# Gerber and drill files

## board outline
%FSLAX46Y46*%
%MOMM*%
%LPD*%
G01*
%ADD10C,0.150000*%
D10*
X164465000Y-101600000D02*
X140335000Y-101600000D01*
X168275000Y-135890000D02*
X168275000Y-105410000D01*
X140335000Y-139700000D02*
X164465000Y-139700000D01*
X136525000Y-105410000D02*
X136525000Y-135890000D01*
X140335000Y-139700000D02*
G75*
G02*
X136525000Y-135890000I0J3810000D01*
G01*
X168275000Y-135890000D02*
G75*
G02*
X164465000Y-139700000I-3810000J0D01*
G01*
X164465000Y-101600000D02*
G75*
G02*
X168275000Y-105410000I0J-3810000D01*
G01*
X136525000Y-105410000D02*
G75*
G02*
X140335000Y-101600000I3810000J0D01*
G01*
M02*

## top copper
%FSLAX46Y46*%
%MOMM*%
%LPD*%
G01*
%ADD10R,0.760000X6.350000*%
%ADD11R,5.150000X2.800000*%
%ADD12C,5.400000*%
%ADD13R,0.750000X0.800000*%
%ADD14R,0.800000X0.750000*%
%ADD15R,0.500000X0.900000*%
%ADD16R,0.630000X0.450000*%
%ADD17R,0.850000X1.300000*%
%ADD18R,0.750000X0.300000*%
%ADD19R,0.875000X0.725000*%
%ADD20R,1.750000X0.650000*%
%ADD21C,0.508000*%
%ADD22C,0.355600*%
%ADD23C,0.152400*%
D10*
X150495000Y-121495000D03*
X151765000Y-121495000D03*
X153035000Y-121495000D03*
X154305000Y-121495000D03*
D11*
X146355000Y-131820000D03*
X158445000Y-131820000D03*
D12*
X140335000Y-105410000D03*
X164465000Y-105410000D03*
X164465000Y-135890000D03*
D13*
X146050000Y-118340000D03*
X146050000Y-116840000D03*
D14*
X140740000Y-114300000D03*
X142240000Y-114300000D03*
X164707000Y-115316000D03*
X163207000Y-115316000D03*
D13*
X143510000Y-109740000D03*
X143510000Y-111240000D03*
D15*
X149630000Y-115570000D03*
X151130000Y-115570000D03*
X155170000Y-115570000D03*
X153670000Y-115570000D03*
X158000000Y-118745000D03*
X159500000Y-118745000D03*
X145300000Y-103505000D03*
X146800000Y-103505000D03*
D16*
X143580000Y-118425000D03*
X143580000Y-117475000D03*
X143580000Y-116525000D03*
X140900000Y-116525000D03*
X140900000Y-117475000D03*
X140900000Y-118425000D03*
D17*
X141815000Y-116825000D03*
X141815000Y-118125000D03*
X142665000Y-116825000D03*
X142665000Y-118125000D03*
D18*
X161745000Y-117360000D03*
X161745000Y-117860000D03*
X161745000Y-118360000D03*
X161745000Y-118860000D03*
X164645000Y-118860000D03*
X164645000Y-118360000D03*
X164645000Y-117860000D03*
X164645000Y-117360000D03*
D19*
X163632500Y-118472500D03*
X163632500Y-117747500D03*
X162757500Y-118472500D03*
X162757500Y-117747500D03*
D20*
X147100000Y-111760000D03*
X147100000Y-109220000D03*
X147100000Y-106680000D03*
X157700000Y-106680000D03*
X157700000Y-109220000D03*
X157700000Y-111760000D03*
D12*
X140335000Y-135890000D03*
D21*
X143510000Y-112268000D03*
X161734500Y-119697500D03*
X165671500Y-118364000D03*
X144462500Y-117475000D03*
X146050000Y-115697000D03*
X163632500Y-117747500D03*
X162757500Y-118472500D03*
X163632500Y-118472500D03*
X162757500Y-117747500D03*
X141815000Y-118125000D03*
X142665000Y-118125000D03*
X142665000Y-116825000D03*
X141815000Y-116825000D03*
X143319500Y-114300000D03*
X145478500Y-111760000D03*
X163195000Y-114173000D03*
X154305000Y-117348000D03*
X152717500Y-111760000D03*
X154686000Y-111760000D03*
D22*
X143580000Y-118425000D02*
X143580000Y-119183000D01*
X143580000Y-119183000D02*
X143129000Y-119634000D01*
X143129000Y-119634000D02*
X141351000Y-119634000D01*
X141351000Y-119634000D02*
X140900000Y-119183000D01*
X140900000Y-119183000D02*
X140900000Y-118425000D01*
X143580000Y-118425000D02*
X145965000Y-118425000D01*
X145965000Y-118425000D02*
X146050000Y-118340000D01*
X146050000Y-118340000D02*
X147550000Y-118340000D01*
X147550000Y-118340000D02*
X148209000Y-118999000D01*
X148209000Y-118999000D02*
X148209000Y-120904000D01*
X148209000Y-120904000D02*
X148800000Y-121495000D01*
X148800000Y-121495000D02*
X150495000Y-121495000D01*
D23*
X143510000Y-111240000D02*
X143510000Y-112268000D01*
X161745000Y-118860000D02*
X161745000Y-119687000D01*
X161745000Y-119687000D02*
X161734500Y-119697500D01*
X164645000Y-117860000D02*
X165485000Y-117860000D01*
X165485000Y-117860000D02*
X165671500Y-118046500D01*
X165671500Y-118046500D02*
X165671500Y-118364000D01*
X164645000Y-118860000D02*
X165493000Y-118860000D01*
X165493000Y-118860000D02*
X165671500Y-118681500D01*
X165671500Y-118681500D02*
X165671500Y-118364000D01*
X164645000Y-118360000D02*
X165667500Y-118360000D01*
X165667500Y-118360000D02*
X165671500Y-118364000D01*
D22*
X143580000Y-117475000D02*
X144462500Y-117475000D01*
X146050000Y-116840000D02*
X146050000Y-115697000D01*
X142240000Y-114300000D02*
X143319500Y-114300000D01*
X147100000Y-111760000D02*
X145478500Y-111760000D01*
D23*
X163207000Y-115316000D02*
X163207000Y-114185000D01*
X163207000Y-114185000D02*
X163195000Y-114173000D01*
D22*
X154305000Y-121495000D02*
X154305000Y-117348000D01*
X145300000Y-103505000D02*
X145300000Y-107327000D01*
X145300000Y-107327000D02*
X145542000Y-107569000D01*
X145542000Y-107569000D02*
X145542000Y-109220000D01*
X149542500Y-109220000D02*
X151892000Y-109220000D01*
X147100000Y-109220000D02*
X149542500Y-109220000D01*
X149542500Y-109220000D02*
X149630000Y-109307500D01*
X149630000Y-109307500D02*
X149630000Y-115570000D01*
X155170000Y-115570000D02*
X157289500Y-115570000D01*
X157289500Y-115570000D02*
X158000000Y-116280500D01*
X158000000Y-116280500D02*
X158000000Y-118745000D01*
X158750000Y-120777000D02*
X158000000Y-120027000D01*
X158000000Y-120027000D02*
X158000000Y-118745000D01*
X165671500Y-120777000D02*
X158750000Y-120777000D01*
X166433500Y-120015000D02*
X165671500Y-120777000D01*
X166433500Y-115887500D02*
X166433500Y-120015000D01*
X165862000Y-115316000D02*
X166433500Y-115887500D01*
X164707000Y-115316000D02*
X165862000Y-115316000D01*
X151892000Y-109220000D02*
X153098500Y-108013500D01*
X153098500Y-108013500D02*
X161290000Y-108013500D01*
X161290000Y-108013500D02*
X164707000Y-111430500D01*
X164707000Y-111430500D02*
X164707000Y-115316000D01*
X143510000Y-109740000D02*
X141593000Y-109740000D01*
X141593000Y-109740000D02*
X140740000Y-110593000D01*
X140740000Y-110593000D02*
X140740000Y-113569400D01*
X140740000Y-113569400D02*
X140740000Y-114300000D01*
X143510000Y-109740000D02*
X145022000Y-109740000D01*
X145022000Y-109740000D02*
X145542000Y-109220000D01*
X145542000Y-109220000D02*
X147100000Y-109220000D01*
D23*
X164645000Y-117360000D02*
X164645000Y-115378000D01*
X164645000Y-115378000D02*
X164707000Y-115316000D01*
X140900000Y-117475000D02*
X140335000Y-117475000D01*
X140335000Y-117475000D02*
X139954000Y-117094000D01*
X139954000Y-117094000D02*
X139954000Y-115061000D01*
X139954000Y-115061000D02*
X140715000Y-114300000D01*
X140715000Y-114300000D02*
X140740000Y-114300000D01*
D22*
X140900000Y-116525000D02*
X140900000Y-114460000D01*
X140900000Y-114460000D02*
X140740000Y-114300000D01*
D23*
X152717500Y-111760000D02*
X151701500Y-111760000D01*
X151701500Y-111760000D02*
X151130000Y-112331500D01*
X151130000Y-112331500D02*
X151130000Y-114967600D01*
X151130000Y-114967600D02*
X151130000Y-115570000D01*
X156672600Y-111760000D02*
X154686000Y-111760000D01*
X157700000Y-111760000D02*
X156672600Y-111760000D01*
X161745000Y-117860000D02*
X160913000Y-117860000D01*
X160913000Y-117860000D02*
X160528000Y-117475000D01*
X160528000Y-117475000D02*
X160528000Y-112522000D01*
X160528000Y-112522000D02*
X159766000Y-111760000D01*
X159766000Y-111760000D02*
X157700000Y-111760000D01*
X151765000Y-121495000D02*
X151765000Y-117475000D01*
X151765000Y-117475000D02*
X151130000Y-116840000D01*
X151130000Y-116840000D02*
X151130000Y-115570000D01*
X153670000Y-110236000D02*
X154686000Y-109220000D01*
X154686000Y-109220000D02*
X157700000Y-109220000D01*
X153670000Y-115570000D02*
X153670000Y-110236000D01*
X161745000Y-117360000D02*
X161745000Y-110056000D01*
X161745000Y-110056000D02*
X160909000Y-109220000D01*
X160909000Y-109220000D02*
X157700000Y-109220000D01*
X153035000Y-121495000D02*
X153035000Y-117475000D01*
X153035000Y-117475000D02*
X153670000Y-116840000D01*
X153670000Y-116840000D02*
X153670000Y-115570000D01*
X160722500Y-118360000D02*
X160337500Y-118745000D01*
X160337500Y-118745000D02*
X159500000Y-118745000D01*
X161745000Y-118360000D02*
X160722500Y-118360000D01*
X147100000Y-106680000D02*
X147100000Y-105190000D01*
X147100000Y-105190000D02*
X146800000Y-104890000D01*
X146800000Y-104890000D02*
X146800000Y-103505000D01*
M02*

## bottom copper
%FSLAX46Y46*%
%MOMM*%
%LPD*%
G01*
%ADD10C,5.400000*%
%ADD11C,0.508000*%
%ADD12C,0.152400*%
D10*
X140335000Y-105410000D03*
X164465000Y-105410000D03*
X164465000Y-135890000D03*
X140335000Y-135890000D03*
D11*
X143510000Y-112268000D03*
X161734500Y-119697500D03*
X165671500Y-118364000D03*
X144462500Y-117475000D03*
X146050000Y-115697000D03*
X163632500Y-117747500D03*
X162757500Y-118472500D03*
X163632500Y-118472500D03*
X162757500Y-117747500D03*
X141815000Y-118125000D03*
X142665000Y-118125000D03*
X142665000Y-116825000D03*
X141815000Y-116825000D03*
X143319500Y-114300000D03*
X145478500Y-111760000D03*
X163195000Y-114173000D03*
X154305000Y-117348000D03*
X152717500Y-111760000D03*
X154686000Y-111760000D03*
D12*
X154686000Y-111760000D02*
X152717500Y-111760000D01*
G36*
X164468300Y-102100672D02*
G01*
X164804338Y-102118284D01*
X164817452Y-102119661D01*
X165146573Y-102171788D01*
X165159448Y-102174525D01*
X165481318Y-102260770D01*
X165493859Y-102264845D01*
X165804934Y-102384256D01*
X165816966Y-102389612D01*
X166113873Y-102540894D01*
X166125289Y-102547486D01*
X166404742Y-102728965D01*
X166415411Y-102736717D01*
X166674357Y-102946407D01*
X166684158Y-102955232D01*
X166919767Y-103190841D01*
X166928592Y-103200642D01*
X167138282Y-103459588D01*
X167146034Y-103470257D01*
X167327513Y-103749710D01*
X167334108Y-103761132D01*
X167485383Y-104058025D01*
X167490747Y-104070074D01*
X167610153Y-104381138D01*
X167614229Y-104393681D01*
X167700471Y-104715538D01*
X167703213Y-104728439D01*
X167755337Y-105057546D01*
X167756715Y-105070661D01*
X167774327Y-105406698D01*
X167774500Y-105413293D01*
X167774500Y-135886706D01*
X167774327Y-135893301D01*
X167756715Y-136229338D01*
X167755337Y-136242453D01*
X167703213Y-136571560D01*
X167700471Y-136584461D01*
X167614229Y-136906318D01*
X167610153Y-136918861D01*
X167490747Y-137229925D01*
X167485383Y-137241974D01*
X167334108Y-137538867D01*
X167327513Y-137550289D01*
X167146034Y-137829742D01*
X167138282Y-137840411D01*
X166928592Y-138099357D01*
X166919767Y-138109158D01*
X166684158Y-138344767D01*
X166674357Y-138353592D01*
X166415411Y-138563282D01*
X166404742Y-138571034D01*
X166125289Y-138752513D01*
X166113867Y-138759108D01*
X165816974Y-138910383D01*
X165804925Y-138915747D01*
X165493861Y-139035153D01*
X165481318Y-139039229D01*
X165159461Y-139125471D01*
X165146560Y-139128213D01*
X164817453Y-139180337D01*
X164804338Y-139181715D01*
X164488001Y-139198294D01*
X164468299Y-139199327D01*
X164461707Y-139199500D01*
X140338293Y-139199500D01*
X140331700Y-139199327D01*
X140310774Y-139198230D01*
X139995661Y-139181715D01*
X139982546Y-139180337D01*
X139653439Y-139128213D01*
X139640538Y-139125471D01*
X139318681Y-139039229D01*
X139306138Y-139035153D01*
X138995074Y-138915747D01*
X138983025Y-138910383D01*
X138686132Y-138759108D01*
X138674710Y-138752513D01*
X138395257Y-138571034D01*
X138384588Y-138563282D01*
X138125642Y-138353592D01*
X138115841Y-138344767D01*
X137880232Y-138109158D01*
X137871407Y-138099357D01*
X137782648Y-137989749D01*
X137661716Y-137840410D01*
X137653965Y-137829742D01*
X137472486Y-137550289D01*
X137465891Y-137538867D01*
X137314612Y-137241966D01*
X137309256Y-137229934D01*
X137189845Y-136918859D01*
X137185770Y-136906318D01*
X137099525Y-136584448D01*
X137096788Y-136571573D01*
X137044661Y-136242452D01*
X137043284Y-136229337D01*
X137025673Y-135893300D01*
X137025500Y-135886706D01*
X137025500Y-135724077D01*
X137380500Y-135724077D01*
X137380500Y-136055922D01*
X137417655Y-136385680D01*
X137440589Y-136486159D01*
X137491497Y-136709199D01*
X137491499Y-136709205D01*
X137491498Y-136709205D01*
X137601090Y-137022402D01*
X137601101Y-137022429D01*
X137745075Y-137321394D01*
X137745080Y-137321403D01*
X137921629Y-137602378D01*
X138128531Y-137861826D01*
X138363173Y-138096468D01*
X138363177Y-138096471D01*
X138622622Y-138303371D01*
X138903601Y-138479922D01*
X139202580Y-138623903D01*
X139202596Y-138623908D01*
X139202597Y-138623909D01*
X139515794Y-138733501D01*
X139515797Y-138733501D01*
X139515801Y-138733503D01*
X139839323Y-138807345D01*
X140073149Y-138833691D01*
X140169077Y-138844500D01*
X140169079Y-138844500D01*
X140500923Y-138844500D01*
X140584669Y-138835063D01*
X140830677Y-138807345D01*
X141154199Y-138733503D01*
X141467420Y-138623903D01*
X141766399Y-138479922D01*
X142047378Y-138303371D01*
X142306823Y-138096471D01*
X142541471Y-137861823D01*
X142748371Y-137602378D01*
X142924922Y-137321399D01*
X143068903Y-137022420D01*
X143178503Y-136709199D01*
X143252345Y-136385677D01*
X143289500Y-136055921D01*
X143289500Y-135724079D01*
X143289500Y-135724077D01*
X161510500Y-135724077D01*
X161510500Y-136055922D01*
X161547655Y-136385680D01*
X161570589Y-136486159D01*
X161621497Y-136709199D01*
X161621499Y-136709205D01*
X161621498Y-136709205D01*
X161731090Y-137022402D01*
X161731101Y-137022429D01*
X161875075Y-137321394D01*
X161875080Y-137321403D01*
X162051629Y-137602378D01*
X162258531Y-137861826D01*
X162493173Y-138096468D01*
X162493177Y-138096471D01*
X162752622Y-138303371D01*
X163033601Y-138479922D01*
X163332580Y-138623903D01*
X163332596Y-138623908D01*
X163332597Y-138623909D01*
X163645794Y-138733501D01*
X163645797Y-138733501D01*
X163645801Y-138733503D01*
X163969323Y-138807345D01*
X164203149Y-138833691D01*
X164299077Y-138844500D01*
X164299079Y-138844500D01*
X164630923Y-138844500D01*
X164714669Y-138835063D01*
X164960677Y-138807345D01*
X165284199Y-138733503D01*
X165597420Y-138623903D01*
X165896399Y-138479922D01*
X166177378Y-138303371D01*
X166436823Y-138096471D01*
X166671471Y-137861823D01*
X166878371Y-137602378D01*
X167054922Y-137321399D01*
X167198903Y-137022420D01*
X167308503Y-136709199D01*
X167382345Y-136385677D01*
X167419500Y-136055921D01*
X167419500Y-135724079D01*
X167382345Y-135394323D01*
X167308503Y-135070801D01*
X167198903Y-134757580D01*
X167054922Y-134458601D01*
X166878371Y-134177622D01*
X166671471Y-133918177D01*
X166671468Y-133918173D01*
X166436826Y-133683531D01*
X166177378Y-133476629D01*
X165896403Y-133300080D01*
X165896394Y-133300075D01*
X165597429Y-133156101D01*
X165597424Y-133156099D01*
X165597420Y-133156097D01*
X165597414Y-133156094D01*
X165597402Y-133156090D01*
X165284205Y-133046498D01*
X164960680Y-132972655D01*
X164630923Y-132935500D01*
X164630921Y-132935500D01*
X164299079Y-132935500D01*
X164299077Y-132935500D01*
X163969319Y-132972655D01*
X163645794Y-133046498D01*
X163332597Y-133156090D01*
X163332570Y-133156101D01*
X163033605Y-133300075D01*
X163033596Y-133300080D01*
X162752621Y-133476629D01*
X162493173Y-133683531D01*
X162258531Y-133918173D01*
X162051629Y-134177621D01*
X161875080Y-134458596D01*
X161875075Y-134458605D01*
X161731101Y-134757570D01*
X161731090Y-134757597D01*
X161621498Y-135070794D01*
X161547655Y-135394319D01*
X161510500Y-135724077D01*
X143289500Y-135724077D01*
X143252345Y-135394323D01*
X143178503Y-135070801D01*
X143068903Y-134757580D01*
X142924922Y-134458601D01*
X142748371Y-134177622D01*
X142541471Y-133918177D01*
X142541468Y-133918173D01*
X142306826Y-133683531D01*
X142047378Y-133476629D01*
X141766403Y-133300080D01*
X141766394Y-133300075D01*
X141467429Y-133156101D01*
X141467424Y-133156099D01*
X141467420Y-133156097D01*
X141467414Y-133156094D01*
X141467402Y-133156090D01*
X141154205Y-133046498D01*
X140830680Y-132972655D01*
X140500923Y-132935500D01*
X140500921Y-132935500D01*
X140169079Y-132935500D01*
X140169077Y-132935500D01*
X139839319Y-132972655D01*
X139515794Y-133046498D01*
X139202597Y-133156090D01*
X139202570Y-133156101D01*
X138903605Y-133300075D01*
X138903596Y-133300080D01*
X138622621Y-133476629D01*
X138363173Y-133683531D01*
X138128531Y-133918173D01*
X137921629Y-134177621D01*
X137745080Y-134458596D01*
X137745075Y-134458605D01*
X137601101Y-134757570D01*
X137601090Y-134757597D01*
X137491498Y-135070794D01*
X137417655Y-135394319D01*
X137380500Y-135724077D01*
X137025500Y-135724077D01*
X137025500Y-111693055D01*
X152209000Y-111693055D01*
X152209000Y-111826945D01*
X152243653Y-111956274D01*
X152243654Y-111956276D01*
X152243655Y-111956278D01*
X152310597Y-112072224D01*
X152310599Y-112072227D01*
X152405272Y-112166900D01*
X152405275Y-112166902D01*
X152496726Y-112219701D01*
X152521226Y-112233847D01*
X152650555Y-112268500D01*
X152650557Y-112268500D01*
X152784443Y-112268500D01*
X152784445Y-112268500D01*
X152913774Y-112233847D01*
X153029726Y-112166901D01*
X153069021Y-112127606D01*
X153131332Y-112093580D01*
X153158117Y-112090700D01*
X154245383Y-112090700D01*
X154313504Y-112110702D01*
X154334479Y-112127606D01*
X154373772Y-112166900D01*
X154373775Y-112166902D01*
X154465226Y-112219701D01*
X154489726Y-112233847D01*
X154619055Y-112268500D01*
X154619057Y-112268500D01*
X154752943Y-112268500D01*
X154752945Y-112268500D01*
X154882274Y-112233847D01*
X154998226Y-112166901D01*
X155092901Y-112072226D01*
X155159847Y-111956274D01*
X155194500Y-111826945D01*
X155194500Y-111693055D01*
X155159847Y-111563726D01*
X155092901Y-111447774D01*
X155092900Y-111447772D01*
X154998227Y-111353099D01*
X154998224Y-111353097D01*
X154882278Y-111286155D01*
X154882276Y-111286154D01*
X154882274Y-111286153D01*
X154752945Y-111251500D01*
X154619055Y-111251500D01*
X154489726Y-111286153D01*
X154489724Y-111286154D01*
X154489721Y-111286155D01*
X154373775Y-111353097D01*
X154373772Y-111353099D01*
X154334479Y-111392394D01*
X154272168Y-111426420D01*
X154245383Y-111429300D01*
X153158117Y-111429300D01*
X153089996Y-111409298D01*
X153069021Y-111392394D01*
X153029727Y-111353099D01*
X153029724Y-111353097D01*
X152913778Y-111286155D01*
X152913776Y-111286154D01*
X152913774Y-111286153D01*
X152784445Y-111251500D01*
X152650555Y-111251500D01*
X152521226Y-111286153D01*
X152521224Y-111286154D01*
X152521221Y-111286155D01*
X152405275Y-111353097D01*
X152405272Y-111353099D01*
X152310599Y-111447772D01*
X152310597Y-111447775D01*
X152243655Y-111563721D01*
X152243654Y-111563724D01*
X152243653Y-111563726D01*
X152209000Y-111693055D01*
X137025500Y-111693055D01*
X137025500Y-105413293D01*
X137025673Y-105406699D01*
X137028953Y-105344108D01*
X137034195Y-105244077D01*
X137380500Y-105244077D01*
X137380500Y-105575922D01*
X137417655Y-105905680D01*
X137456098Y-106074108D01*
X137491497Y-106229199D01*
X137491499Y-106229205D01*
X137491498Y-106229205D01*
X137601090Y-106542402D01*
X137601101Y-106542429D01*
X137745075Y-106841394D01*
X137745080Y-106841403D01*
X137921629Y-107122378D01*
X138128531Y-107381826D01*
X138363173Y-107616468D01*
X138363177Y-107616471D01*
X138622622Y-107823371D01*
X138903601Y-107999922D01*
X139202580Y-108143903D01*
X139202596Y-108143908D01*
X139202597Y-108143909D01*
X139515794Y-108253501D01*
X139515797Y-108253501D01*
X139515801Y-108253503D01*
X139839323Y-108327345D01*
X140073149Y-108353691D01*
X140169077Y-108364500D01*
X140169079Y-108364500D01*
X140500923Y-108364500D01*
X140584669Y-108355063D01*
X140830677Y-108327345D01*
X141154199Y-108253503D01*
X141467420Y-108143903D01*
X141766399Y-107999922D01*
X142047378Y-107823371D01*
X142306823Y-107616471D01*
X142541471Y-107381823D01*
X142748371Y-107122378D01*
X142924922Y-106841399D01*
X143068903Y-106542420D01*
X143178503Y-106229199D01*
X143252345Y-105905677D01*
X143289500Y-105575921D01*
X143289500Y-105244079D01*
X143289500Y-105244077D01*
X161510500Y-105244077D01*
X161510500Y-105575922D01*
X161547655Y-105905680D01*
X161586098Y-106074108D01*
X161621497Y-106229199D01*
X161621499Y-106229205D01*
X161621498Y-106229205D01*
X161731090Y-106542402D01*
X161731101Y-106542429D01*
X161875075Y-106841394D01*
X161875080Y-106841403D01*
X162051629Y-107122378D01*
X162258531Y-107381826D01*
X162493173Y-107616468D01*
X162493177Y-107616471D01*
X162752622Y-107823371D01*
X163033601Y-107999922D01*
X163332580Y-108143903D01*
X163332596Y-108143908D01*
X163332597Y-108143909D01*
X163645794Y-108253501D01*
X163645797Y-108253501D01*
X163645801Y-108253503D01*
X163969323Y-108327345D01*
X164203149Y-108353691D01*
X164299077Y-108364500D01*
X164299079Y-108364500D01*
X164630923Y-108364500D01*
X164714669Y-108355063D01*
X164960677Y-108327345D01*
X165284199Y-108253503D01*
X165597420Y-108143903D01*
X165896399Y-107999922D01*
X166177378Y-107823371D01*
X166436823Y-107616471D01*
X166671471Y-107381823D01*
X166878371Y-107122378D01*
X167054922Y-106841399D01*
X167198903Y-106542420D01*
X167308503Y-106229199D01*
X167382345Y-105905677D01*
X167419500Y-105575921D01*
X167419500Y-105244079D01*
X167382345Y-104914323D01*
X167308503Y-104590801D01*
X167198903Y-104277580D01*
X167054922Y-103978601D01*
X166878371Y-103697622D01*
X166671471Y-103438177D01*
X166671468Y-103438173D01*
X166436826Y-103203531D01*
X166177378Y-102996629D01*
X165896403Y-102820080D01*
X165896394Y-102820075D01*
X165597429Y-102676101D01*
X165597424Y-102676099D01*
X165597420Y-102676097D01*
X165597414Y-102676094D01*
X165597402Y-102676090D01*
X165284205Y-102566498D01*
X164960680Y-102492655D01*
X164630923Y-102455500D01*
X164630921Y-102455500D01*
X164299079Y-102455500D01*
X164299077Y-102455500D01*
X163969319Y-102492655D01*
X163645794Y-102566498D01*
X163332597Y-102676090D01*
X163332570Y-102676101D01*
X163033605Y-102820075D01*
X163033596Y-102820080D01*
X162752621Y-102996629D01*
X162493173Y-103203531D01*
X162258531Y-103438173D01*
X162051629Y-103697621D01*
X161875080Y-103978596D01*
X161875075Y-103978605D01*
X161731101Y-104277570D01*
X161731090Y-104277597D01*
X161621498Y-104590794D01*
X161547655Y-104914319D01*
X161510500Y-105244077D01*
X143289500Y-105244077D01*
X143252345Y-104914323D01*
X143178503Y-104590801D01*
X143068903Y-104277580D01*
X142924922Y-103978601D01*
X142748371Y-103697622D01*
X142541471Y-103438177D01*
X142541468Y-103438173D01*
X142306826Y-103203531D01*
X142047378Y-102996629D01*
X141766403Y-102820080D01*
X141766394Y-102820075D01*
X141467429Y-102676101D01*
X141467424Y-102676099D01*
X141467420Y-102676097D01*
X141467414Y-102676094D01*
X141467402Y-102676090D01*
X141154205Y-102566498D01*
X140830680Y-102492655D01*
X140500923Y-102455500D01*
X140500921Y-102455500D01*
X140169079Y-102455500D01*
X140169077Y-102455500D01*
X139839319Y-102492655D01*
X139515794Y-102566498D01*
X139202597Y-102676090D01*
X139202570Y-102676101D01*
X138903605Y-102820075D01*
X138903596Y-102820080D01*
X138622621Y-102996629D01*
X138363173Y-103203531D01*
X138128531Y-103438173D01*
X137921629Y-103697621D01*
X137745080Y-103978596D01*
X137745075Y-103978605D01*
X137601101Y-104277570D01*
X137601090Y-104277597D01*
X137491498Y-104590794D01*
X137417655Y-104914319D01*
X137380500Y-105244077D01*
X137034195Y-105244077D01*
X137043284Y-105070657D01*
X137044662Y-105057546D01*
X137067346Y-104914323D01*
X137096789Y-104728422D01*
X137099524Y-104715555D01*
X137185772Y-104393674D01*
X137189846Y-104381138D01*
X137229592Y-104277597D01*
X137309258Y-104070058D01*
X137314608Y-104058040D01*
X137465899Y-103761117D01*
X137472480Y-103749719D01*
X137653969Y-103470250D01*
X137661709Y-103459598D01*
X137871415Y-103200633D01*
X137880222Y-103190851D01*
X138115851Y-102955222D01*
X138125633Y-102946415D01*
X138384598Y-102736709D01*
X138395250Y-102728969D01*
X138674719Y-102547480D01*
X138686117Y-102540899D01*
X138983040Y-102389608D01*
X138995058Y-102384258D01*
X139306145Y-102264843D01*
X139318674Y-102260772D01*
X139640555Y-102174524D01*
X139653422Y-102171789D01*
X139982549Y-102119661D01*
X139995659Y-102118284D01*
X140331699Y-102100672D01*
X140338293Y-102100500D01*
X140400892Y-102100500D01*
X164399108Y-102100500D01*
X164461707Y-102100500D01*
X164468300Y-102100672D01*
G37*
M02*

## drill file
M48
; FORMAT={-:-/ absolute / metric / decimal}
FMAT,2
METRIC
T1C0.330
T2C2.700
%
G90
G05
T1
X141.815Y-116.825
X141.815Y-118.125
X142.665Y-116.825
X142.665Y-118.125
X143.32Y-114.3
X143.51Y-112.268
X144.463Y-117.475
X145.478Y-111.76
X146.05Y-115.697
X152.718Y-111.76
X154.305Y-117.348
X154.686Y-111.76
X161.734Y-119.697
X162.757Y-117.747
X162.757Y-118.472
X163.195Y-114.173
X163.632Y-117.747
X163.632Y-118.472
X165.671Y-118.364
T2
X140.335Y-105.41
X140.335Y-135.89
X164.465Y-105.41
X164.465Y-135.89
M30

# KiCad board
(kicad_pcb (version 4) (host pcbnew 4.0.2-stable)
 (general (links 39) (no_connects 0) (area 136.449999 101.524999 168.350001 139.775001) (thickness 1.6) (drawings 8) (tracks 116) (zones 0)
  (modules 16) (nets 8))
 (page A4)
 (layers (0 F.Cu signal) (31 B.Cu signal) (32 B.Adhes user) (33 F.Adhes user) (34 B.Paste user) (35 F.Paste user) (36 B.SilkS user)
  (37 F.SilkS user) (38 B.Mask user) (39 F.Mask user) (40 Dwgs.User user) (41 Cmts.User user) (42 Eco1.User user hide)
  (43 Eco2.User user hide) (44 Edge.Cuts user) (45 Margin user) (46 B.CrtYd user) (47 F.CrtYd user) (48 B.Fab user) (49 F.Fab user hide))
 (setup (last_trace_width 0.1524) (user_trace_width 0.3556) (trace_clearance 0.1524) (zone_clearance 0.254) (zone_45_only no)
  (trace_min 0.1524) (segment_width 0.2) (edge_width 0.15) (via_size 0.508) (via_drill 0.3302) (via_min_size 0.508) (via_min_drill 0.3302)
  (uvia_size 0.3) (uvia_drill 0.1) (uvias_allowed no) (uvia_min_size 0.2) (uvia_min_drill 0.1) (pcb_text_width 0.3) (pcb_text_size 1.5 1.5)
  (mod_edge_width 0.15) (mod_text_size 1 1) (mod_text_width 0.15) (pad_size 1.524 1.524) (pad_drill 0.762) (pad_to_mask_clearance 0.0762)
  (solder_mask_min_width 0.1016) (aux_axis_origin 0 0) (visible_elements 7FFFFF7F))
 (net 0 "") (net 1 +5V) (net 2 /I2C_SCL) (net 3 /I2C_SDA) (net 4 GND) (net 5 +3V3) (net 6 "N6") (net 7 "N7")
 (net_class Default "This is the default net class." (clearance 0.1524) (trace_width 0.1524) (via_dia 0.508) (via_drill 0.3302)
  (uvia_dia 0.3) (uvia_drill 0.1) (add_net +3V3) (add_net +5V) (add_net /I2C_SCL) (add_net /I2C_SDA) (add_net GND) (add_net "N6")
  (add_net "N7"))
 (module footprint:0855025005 (layer F.Cu) (at 152.4 139.7)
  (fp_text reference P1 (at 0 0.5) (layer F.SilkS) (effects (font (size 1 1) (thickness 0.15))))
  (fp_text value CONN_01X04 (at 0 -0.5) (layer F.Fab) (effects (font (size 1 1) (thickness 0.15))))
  (pad 1 smd rect (at -1.905 -18.205) (size 0.76 6.35) (layers F.Cu F.Paste F.Mask) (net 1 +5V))
  (pad 2 smd rect (at -0.635 -18.205) (size 0.76 6.35) (layers F.Cu F.Paste F.Mask) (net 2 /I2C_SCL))
  (pad 3 smd rect (at 0.635 -18.205) (size 0.76 6.35) (layers F.Cu F.Paste F.Mask) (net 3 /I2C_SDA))
  (pad 4 smd rect (at 1.905 -18.205) (size 0.76 6.35) (layers F.Cu F.Paste F.Mask) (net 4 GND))
  (pad 5 smd rect (at -6.045 -7.88) (size 5.15 2.8) (layers F.Cu F.Paste F.Mask))
  (pad 5 smd rect (at 6.045 -7.88) (size 5.15 2.8) (layers F.Cu F.Paste F.Mask)))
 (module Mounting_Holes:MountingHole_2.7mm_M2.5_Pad (layer F.Cu) (at 140.335 105.41)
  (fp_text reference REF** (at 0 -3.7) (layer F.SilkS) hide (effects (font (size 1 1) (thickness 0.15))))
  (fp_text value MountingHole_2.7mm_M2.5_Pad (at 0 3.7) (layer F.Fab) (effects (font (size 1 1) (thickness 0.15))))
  (pad 1 thru_hole circle (at 0 0) (size 5.4 5.4) (drill 2.7) (layers *.Cu *.Mask F.SilkS)))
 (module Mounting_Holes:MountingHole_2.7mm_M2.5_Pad (layer F.Cu) (at 164.465 105.41)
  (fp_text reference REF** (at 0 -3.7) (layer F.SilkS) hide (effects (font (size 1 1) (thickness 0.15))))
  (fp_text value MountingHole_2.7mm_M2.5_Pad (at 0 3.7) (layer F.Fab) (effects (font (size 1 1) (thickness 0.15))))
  (pad 1 thru_hole circle (at 0 0) (size 5.4 5.4) (drill 2.7) (layers *.Cu *.Mask F.SilkS)))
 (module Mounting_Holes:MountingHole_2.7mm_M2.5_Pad (layer F.Cu) (at 164.465 135.89)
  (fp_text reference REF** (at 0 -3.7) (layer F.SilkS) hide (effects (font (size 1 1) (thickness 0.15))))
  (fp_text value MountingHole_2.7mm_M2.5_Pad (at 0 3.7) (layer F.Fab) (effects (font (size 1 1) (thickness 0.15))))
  (pad 1 thru_hole circle (at 0 0) (size 5.4 5.4) (drill 2.7) (layers *.Cu *.Mask F.SilkS)))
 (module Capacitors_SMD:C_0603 (layer F.Cu) (at 146.05 117.59 90)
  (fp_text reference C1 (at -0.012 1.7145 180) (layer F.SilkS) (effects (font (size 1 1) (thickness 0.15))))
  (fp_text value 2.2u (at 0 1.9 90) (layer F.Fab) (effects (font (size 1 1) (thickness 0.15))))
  (pad 1 smd rect (at -0.75 0 90) (size 0.8 0.75) (layers F.Cu F.Paste F.Mask) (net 1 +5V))
  (pad 2 smd rect (at 0.75 0 90) (size 0.8 0.75) (layers F.Cu F.Paste F.Mask) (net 4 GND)))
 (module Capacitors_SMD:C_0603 (layer F.Cu) (at 141.49 114.3)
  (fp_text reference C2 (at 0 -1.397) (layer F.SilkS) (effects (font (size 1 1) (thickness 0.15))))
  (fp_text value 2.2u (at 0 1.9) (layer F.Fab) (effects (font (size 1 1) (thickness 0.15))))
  (pad 1 smd rect (at -0.75 0) (size 0.8 0.75) (layers F.Cu F.Paste F.Mask) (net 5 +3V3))
  (pad 2 smd rect (at 0.75 0) (size 0.8 0.75) (layers F.Cu F.Paste F.Mask) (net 4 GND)))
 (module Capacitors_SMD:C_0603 (layer F.Cu) (at 163.957 115.316 180)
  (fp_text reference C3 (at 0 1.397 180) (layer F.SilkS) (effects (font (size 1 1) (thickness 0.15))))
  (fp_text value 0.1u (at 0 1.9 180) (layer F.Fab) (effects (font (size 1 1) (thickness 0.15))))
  (pad 1 smd rect (at -0.75 0 180) (size 0.8 0.75) (layers F.Cu F.Paste F.Mask) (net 5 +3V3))
  (pad 2 smd rect (at 0.75 0 180) (size 0.8 0.75) (layers F.Cu F.Paste F.Mask) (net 4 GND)))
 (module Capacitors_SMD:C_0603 (layer F.Cu) (at 143.51 110.49 270)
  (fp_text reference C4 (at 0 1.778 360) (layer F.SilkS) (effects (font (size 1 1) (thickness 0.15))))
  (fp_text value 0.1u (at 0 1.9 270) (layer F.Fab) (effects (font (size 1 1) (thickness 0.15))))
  (pad 1 smd rect (at -0.75 0 270) (size 0.8 0.75) (layers F.Cu F.Paste F.Mask) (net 5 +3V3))
  (pad 2 smd rect (at 0.75 0 270) (size 0.8 0.75) (layers F.Cu F.Paste F.Mask) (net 4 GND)))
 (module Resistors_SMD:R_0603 (layer F.Cu) (at 150.38 115.57)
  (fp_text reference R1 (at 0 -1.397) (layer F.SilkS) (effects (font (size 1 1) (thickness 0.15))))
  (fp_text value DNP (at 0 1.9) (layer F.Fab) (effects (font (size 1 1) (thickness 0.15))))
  (pad 1 smd rect (at -0.75 0) (size 0.5 0.9) (layers F.Cu F.Paste F.Mask) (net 5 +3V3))
  (pad 2 smd rect (at 0.75 0) (size 0.5 0.9) (layers F.Cu F.Paste F.Mask) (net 2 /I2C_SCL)))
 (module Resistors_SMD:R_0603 (layer F.Cu) (at 154.42 115.57 180)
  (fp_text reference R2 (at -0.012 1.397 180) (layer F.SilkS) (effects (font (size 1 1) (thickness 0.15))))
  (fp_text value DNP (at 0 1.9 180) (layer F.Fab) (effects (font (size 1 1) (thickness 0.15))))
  (pad 1 smd rect (at -0.75 0 180) (size 0.5 0.9) (layers F.Cu F.Paste F.Mask) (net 5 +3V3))
  (pad 2 smd rect (at 0.75 0 180) (size 0.5 0.9) (layers F.Cu F.Paste F.Mask) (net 3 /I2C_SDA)))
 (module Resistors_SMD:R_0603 (layer F.Cu) (at 158.75 118.745)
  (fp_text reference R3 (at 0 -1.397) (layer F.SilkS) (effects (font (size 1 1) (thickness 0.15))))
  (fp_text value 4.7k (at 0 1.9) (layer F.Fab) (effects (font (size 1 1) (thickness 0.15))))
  (pad 1 smd rect (at -0.75 0) (size 0.5 0.9) (layers F.Cu F.Paste F.Mask) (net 5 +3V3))
  (pad 2 smd rect (at 0.75 0) (size 0.5 0.9) (layers F.Cu F.Paste F.Mask) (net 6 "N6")))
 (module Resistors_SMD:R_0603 (layer F.Cu) (at 146.05 103.505)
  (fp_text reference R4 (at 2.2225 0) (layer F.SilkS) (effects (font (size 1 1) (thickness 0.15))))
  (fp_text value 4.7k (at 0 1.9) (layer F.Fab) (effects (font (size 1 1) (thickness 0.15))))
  (pad 1 smd rect (at -0.75 0) (size 0.5 0.9) (layers F.Cu F.Paste F.Mask) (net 5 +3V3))
  (pad 2 smd rect (at 0.75 0) (size 0.5 0.9) (layers F.Cu F.Paste F.Mask) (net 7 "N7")))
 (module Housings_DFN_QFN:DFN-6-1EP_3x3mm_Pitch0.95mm (layer F.Cu) (at 142.24 117.475 180)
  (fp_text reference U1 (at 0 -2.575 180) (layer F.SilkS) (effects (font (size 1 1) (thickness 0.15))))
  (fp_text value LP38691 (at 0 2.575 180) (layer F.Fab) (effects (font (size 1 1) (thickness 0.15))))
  (pad 1 smd rect (at -1.34 -0.95 180) (size 0.63 0.45) (layers F.Cu F.Paste F.Mask) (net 1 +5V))
  (pad 2 smd rect (at -1.34 0 180) (size 0.63 0.45) (layers F.Cu F.Paste F.Mask) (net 4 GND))
  (pad 3 smd rect (at -1.34 0.95 180) (size 0.63 0.45) (layers F.Cu F.Paste F.Mask))
  (pad 4 smd rect (at 1.34 0.95 180) (size 0.63 0.45) (layers F.Cu F.Paste F.Mask) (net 5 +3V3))
  (pad 5 smd rect (at 1.34 0 180) (size 0.63 0.45) (layers F.Cu F.Paste F.Mask) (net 5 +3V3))
  (pad 6 smd rect (at 1.34 -0.95 180) (size 0.63 0.45) (layers F.Cu F.Paste F.Mask) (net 1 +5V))
  (pad 7 smd rect (at 0.425 0.65 180) (size 0.85 1.3) (layers F.Cu F.Paste F.Mask) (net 4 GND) (solder_paste_margin_ratio -0.2))
  (pad 7 smd rect (at 0.425 -0.65 180) (size 0.85 1.3) (layers F.Cu F.Paste F.Mask) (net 4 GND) (solder_paste_margin_ratio -0.2))
  (pad 7 smd rect (at -0.425 0.65 180) (size 0.85 1.3) (layers F.Cu F.Paste F.Mask) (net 4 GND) (solder_paste_margin_ratio -0.2))
  (pad 7 smd rect (at -0.425 -0.65 180) (size 0.85 1.3) (layers F.Cu F.Paste F.Mask) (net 4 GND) (solder_paste_margin_ratio -0.2)))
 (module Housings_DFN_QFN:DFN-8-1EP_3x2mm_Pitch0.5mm (layer F.Cu) (at 163.195 118.11)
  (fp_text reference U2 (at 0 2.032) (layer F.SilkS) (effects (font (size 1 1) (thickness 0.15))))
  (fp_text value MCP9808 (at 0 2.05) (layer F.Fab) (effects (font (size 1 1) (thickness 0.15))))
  (pad 1 smd rect (at -1.45 -0.75) (size 0.75 0.3) (layers F.Cu F.Paste F.Mask) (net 3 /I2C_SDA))
  (pad 2 smd rect (at -1.45 -0.25) (size 0.75 0.3) (layers F.Cu F.Paste F.Mask) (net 2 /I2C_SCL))
  (pad 3 smd rect (at -1.45 0.25) (size 0.75 0.3) (layers F.Cu F.Paste F.Mask) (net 6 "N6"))
  (pad 4 smd rect (at -1.45 0.75) (size 0.75 0.3) (layers F.Cu F.Paste F.Mask) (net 4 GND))
  (pad 5 smd rect (at 1.45 0.75) (size 0.75 0.3) (layers F.Cu F.Paste F.Mask) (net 4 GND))
  (pad 6 smd rect (at 1.45 0.25) (size 0.75 0.3) (layers F.Cu F.Paste F.Mask) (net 4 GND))
  (pad 7 smd rect (at 1.45 -0.25) (size 0.75 0.3) (layers F.Cu F.Paste F.Mask) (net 4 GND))
  (pad 8 smd rect (at 1.45 -0.75) (size 0.75 0.3) (layers F.Cu F.Paste F.Mask) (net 5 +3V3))
  (pad 9 smd rect (at 0.4375 0.3625) (size 0.875 0.725) (layers F.Cu F.Paste F.Mask) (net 4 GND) (solder_paste_margin_ratio -0.2))
  (pad 9 smd rect (at 0.4375 -0.3625) (size 0.875 0.725) (layers F.Cu F.Paste F.Mask) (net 4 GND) (solder_paste_margin_ratio -0.2))
  (pad 9 smd rect (at -0.4375 0.3625) (size 0.875 0.725) (layers F.Cu F.Paste F.Mask) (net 4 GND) (solder_paste_margin_ratio -0.2))
  (pad 9 smd rect (at -0.4375 -0.3625) (size 0.875 0.725) (layers F.Cu F.Paste F.Mask) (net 4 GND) (solder_paste_margin_ratio -0.2)))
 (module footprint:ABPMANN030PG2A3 (layer F.Cu) (at 152.4 109.22)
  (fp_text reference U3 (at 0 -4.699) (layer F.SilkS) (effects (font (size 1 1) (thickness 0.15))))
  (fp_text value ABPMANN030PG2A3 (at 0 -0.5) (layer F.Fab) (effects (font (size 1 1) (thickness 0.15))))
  (pad 1 smd rect (at -5.3 2.54) (size 1.75 0.65) (layers F.Cu F.Paste F.Mask) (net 4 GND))
  (pad 2 smd rect (at -5.3 0) (size 1.75 0.65) (layers F.Cu F.Paste F.Mask) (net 5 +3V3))
  (pad 3 smd rect (at -5.3 -2.54) (size 1.75 0.65) (layers F.Cu F.Paste F.Mask) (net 7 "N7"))
  (pad 4 smd rect (at 5.3 -2.54) (size 1.75 0.65) (layers F.Cu F.Paste F.Mask))
  (pad 5 smd rect (at 5.3 0) (size 1.75 0.65) (layers F.Cu F.Paste F.Mask) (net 3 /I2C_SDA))
  (pad 6 smd rect (at 5.3 2.54) (size 1.75 0.65) (layers F.Cu F.Paste F.Mask) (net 2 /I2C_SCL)))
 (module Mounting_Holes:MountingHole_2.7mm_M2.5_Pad (layer F.Cu) (at 140.335 135.89)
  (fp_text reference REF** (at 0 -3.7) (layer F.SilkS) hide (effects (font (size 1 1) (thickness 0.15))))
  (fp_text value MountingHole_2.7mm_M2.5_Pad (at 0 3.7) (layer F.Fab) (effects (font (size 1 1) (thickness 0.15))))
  (pad 1 thru_hole circle (at 0 0) (size 5.4 5.4) (drill 2.7) (layers *.Cu *.Mask F.SilkS)))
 (gr_line (start 164.465 101.6) (end 140.335 101.6) (layer Edge.Cuts) (width 0.15))
 (gr_line (start 168.275 135.89) (end 168.275 105.41) (layer Edge.Cuts) (width 0.15))
 (gr_line (start 140.335 139.7) (end 164.465 139.7) (layer Edge.Cuts) (width 0.15))
 (gr_line (start 136.525 105.41) (end 136.525 135.89) (layer Edge.Cuts) (width 0.15))
 (gr_arc (start 140.335 135.89) (end 140.335 139.7) (angle 90) (layer Edge.Cuts) (width 0.15))
 (gr_arc (start 164.465 135.89) (end 168.275 135.89) (angle 90) (layer Edge.Cuts) (width 0.15))
 (gr_arc (start 164.465 105.41) (end 164.465 101.6) (angle 90) (layer Edge.Cuts) (width 0.15))
 (gr_arc (start 140.335 105.41) (end 136.525 105.41) (angle 90) (layer Edge.Cuts) (width 0.15))
 (segment (start 143.58 118.425) (end 143.58 119.183) (width 0.3556) (layer F.Cu) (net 1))
 (segment (start 143.58 119.183) (end 143.129 119.634) (width 0.3556) (layer F.Cu) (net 1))
 (segment (start 143.129 119.634) (end 141.351 119.634) (width 0.3556) (layer F.Cu) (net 1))
 (segment (start 141.351 119.634) (end 140.9 119.183) (width 0.3556) (layer F.Cu) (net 1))
 (segment (start 140.9 119.183) (end 140.9 118.425) (width 0.3556) (layer F.Cu) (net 1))
 (segment (start 143.58 118.425) (end 145.965 118.425) (width 0.3556) (layer F.Cu) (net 1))
 (segment (start 145.965 118.425) (end 146.05 118.34) (width 0.3556) (layer F.Cu) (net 1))
 (segment (start 146.05 118.34) (end 147.55 118.34) (width 0.3556) (layer F.Cu) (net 1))
 (segment (start 147.55 118.34) (end 148.209 118.999) (width 0.3556) (layer F.Cu) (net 1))
 (segment (start 148.209 118.999) (end 148.209 120.904) (width 0.3556) (layer F.Cu) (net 1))
 (segment (start 148.209 120.904) (end 148.8 121.495) (width 0.3556) (layer F.Cu) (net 1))
 (segment (start 148.8 121.495) (end 150.495 121.495) (width 0.3556) (layer F.Cu) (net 1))
 (segment (start 143.51 111.24) (end 143.51 112.268) (width 0.1524) (layer F.Cu) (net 4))
 (via (at 143.51 112.268) (size 0.508) (drill 0.3302) (layers F.Cu B.Cu) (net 4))
 (segment (start 161.745 118.86) (end 161.745 119.687) (width 0.1524) (layer F.Cu) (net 4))
 (segment (start 161.745 119.687) (end 161.7345 119.6975) (width 0.1524) (layer F.Cu) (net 4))
 (via (at 161.7345 119.6975) (size 0.508) (drill 0.3302) (layers F.Cu B.Cu) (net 4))
 (segment (start 164.645 117.86) (end 165.485 117.86) (width 0.1524) (layer F.Cu) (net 4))
 (segment (start 165.485 117.86) (end 165.6715 118.0465) (width 0.1524) (layer F.Cu) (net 4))
 (segment (start 165.6715 118.0465) (end 165.6715 118.364) (width 0.1524) (layer F.Cu) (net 4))
 (segment (start 164.645 118.86) (end 165.493 118.86) (width 0.1524) (layer F.Cu) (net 4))
 (segment (start 165.493 118.86) (end 165.6715 118.6815) (width 0.1524) (layer F.Cu) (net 4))
 (segment (start 165.6715 118.6815) (end 165.6715 118.364) (width 0.1524) (layer F.Cu) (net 4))
 (segment (start 164.645 118.36) (end 165.6675 118.36) (width 0.1524) (layer F.Cu) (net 4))
 (segment (start 165.6675 118.36) (end 165.6715 118.364) (width 0.1524) (layer F.Cu) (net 4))
 (via (at 165.6715 118.364) (size 0.508) (drill 0.3302) (layers F.Cu B.Cu) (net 4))
 (segment (start 143.58 117.475) (end 144.4625 117.475) (width 0.3556) (layer F.Cu) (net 4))
 (via (at 144.4625 117.475) (size 0.508) (drill 0.3302) (layers F.Cu B.Cu) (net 4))
 (segment (start 146.05 116.84) (end 146.05 115.697) (width 0.3556) (layer F.Cu) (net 4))
 (via (at 146.05 115.697) (size 0.508) (drill 0.3302) (layers F.Cu B.Cu) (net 4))
 (via (at 163.6325 117.7475) (size 0.508) (drill 0.3302) (layers F.Cu B.Cu) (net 4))
 (via (at 162.7575 118.4725) (size 0.508) (drill 0.3302) (layers F.Cu B.Cu) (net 4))
 (via (at 163.6325 118.4725) (size 0.508) (drill 0.3302) (layers F.Cu B.Cu) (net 4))
 (via (at 162.7575 117.7475) (size 0.508) (drill 0.3302) (layers F.Cu B.Cu) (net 4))
 (via (at 141.815 118.125) (size 0.508) (drill 0.3302) (layers F.Cu B.Cu) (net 4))
 (via (at 142.665 118.125) (size 0.508) (drill 0.3302) (layers F.Cu B.Cu) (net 4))
 (via (at 142.665 116.825) (size 0.508) (drill 0.3302) (layers F.Cu B.Cu) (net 4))
 (via (at 141.815 116.825) (size 0.508) (drill 0.3302) (layers F.Cu B.Cu) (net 4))
 (segment (start 142.24 114.3) (end 143.3195 114.3) (width 0.3556) (layer F.Cu) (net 4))
 (via (at 143.3195 114.3) (size 0.508) (drill 0.3302) (layers F.Cu B.Cu) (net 4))
 (segment (start 147.1 111.76) (end 145.4785 111.76) (width 0.3556) (layer F.Cu) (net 4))
 (via (at 145.4785 111.76) (size 0.508) (drill 0.3302) (layers F.Cu B.Cu) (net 4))
 (segment (start 163.207 115.316) (end 163.207 114.185) (width 0.1524) (layer F.Cu) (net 4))
 (segment (start 163.207 114.185) (end 163.195 114.173) (width 0.1524) (layer F.Cu) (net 4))
 (via (at 163.195 114.173) (size 0.508) (drill 0.3302) (layers F.Cu B.Cu) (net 4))
 (segment (start 154.305 121.495) (end 154.305 117.348) (width 0.3556) (layer F.Cu) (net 4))
 (via (at 154.305 117.348) (size 0.508) (drill 0.3302) (layers F.Cu B.Cu) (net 4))
 (segment (start 145.3 103.505) (end 145.3 107.327) (width 0.3556) (layer F.Cu) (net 5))
 (segment (start 145.3 107.327) (end 145.542 107.569) (width 0.3556) (layer F.Cu) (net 5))
 (segment (start 145.542 107.569) (end 145.542 109.22) (width 0.3556) (layer F.Cu) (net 5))
 (segment (start 149.5425 109.22) (end 151.892 109.22) (width 0.3556) (layer F.Cu) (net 5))
 (segment (start 147.1 109.22) (end 149.5425 109.22) (width 0.3556) (layer F.Cu) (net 5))
 (segment (start 149.5425 109.22) (end 149.63 109.3075) (width 0.3556) (layer F.Cu) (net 5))
 (segment (start 149.63 109.3075) (end 149.63 115.57) (width 0.3556) (layer F.Cu) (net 5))
 (segment (start 155.17 115.57) (end 157.2895 115.57) (width 0.3556) (layer F.Cu) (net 5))
 (segment (start 157.2895 115.57) (end 158 116.2805) (width 0.3556) (layer F.Cu) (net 5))
 (segment (start 158 116.2805) (end 158 118.745) (width 0.3556) (layer F.Cu) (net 5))
 (segment (start 158.75 120.777) (end 158 120.027) (width 0.3556) (layer F.Cu) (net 5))
 (segment (start 158 120.027) (end 158 118.745) (width 0.3556) (layer F.Cu) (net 5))
 (segment (start 165.6715 120.777) (end 158.75 120.777) (width 0.3556) (layer F.Cu) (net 5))
 (segment (start 166.4335 120.015) (end 165.6715 120.777) (width 0.3556) (layer F.Cu) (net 5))
 (segment (start 166.4335 115.8875) (end 166.4335 120.015) (width 0.3556) (layer F.Cu) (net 5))
 (segment (start 165.862 115.316) (end 166.4335 115.8875) (width 0.3556) (layer F.Cu) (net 5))
 (segment (start 164.707 115.316) (end 165.862 115.316) (width 0.3556) (layer F.Cu) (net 5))
 (segment (start 151.892 109.22) (end 153.0985 108.0135) (width 0.3556) (layer F.Cu) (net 5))
 (segment (start 153.0985 108.0135) (end 161.29 108.0135) (width 0.3556) (layer F.Cu) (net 5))
 (segment (start 161.29 108.0135) (end 164.707 111.4305) (width 0.3556) (layer F.Cu) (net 5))
 (segment (start 164.707 111.4305) (end 164.707 115.316) (width 0.3556) (layer F.Cu) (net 5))
 (segment (start 143.51 109.74) (end 141.593 109.74) (width 0.3556) (layer F.Cu) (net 5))
 (segment (start 141.593 109.74) (end 140.74 110.593) (width 0.3556) (layer F.Cu) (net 5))
 (segment (start 140.74 110.593) (end 140.74 113.5694) (width 0.3556) (layer F.Cu) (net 5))
 (segment (start 140.74 113.5694) (end 140.74 114.3) (width 0.3556) (layer F.Cu) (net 5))
 (segment (start 143.51 109.74) (end 145.022 109.74) (width 0.3556) (layer F.Cu) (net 5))
 (segment (start 145.022 109.74) (end 145.542 109.22) (width 0.3556) (layer F.Cu) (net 5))
 (segment (start 145.542 109.22) (end 147.1 109.22) (width 0.3556) (layer F.Cu) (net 5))
 (segment (start 164.645 117.36) (end 164.645 115.378) (width 0.1524) (layer F.Cu) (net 5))
 (segment (start 164.645 115.378) (end 164.707 115.316) (width 0.1524) (layer F.Cu) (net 5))
 (segment (start 140.9 117.475) (end 140.335 117.475) (width 0.1524) (layer F.Cu) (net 5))
 (segment (start 140.335 117.475) (end 139.954 117.094) (width 0.1524) (layer F.Cu) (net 5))
 (segment (start 139.954 117.094) (end 139.954 115.061) (width 0.1524) (layer F.Cu) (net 5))
 (segment (start 139.954 115.061) (end 140.715 114.3) (width 0.1524) (layer F.Cu) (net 5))
 (segment (start 140.715 114.3) (end 140.74 114.3) (width 0.1524) (layer F.Cu) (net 5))
 (segment (start 140.9 116.525) (end 140.9 114.46) (width 0.3556) (layer F.Cu) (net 5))
 (segment (start 140.9 114.46) (end 140.74 114.3) (width 0.3556) (layer F.Cu) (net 5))
 (segment (start 152.7175 111.76) (end 151.7015 111.76) (width 0.1524) (layer F.Cu) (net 2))
 (segment (start 151.7015 111.76) (end 151.13 112.3315) (width 0.1524) (layer F.Cu) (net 2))
 (segment (start 151.13 112.3315) (end 151.13 114.9676) (width 0.1524) (layer F.Cu) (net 2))
 (segment (start 151.13 114.9676) (end 151.13 115.57) (width 0.1524) (layer F.Cu) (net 2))
 (segment (start 154.686 111.76) (end 152.7175 111.76) (width 0.1524) (layer B.Cu) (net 2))
 (via (at 152.7175 111.76) (size 0.508) (drill 0.3302) (layers F.Cu B.Cu) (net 2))
 (segment (start 156.6726 111.76) (end 154.686 111.76) (width 0.1524) (layer F.Cu) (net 2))
 (via (at 154.686 111.76) (size 0.508) (drill 0.3302) (layers F.Cu B.Cu) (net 2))
 (segment (start 157.7 111.76) (end 156.6726 111.76) (width 0.1524) (layer F.Cu) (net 2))
 (segment (start 161.745 117.86) (end 160.913 117.86) (width 0.1524) (layer F.Cu) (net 2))
 (segment (start 160.913 117.86) (end 160.528 117.475) (width 0.1524) (layer F.Cu) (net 2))
 (segment (start 160.528 117.475) (end 160.528 112.522) (width 0.1524) (layer F.Cu) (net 2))
 (segment (start 160.528 112.522) (end 159.766 111.76) (width 0.1524) (layer F.Cu) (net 2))
 (segment (start 159.766 111.76) (end 157.7 111.76) (width 0.1524) (layer F.Cu) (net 2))
 (segment (start 151.765 121.495) (end 151.765 117.475) (width 0.1524) (layer F.Cu) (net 2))
 (segment (start 151.765 117.475) (end 151.13 116.84) (width 0.1524) (layer F.Cu) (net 2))
 (segment (start 151.13 116.84) (end 151.13 115.57) (width 0.1524) (layer F.Cu) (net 2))
 (segment (start 153.67 110.236) (end 154.686 109.22) (width 0.1524) (layer F.Cu) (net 3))
 (segment (start 154.686 109.22) (end 157.7 109.22) (width 0.1524) (layer F.Cu) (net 3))
 (segment (start 153.67 115.57) (end 153.67 110.236) (width 0.1524) (layer F.Cu) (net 3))
 (segment (start 161.745 117.36) (end 161.745 110.056) (width 0.1524) (layer F.Cu) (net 3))
 (segment (start 161.745 110.056) (end 160.909 109.22) (width 0.1524) (layer F.Cu) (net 3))
 (segment (start 160.909 109.22) (end 157.7 109.22) (width 0.1524) (layer F.Cu) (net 3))
 (segment (start 153.035 121.495) (end 153.035 117.475) (width 0.1524) (layer F.Cu) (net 3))
 (segment (start 153.035 117.475) (end 153.67 116.84) (width 0.1524) (layer F.Cu) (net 3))
 (segment (start 153.67 116.84) (end 153.67 115.57) (width 0.1524) (layer F.Cu) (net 3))
 (segment (start 160.7225 118.36) (end 160.3375 118.745) (width 0.1524) (layer F.Cu) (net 6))
 (segment (start 160.3375 118.745) (end 159.5 118.745) (width 0.1524) (layer F.Cu) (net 6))
 (segment (start 161.745 118.36) (end 160.7225 118.36) (width 0.1524) (layer F.Cu) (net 6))
 (segment (start 147.1 106.68) (end 147.1 105.19) (width 0.1524) (layer F.Cu) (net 7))
 (segment (start 147.1 105.19) (end 146.8 104.89) (width 0.1524) (layer F.Cu) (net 7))
 (segment (start 146.8 104.89) (end 146.8 103.505) (width 0.1524) (layer F.Cu) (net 7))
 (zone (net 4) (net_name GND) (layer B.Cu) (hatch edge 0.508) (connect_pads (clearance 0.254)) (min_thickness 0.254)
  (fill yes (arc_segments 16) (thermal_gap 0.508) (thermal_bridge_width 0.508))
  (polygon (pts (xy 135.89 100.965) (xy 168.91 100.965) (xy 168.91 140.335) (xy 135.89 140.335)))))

